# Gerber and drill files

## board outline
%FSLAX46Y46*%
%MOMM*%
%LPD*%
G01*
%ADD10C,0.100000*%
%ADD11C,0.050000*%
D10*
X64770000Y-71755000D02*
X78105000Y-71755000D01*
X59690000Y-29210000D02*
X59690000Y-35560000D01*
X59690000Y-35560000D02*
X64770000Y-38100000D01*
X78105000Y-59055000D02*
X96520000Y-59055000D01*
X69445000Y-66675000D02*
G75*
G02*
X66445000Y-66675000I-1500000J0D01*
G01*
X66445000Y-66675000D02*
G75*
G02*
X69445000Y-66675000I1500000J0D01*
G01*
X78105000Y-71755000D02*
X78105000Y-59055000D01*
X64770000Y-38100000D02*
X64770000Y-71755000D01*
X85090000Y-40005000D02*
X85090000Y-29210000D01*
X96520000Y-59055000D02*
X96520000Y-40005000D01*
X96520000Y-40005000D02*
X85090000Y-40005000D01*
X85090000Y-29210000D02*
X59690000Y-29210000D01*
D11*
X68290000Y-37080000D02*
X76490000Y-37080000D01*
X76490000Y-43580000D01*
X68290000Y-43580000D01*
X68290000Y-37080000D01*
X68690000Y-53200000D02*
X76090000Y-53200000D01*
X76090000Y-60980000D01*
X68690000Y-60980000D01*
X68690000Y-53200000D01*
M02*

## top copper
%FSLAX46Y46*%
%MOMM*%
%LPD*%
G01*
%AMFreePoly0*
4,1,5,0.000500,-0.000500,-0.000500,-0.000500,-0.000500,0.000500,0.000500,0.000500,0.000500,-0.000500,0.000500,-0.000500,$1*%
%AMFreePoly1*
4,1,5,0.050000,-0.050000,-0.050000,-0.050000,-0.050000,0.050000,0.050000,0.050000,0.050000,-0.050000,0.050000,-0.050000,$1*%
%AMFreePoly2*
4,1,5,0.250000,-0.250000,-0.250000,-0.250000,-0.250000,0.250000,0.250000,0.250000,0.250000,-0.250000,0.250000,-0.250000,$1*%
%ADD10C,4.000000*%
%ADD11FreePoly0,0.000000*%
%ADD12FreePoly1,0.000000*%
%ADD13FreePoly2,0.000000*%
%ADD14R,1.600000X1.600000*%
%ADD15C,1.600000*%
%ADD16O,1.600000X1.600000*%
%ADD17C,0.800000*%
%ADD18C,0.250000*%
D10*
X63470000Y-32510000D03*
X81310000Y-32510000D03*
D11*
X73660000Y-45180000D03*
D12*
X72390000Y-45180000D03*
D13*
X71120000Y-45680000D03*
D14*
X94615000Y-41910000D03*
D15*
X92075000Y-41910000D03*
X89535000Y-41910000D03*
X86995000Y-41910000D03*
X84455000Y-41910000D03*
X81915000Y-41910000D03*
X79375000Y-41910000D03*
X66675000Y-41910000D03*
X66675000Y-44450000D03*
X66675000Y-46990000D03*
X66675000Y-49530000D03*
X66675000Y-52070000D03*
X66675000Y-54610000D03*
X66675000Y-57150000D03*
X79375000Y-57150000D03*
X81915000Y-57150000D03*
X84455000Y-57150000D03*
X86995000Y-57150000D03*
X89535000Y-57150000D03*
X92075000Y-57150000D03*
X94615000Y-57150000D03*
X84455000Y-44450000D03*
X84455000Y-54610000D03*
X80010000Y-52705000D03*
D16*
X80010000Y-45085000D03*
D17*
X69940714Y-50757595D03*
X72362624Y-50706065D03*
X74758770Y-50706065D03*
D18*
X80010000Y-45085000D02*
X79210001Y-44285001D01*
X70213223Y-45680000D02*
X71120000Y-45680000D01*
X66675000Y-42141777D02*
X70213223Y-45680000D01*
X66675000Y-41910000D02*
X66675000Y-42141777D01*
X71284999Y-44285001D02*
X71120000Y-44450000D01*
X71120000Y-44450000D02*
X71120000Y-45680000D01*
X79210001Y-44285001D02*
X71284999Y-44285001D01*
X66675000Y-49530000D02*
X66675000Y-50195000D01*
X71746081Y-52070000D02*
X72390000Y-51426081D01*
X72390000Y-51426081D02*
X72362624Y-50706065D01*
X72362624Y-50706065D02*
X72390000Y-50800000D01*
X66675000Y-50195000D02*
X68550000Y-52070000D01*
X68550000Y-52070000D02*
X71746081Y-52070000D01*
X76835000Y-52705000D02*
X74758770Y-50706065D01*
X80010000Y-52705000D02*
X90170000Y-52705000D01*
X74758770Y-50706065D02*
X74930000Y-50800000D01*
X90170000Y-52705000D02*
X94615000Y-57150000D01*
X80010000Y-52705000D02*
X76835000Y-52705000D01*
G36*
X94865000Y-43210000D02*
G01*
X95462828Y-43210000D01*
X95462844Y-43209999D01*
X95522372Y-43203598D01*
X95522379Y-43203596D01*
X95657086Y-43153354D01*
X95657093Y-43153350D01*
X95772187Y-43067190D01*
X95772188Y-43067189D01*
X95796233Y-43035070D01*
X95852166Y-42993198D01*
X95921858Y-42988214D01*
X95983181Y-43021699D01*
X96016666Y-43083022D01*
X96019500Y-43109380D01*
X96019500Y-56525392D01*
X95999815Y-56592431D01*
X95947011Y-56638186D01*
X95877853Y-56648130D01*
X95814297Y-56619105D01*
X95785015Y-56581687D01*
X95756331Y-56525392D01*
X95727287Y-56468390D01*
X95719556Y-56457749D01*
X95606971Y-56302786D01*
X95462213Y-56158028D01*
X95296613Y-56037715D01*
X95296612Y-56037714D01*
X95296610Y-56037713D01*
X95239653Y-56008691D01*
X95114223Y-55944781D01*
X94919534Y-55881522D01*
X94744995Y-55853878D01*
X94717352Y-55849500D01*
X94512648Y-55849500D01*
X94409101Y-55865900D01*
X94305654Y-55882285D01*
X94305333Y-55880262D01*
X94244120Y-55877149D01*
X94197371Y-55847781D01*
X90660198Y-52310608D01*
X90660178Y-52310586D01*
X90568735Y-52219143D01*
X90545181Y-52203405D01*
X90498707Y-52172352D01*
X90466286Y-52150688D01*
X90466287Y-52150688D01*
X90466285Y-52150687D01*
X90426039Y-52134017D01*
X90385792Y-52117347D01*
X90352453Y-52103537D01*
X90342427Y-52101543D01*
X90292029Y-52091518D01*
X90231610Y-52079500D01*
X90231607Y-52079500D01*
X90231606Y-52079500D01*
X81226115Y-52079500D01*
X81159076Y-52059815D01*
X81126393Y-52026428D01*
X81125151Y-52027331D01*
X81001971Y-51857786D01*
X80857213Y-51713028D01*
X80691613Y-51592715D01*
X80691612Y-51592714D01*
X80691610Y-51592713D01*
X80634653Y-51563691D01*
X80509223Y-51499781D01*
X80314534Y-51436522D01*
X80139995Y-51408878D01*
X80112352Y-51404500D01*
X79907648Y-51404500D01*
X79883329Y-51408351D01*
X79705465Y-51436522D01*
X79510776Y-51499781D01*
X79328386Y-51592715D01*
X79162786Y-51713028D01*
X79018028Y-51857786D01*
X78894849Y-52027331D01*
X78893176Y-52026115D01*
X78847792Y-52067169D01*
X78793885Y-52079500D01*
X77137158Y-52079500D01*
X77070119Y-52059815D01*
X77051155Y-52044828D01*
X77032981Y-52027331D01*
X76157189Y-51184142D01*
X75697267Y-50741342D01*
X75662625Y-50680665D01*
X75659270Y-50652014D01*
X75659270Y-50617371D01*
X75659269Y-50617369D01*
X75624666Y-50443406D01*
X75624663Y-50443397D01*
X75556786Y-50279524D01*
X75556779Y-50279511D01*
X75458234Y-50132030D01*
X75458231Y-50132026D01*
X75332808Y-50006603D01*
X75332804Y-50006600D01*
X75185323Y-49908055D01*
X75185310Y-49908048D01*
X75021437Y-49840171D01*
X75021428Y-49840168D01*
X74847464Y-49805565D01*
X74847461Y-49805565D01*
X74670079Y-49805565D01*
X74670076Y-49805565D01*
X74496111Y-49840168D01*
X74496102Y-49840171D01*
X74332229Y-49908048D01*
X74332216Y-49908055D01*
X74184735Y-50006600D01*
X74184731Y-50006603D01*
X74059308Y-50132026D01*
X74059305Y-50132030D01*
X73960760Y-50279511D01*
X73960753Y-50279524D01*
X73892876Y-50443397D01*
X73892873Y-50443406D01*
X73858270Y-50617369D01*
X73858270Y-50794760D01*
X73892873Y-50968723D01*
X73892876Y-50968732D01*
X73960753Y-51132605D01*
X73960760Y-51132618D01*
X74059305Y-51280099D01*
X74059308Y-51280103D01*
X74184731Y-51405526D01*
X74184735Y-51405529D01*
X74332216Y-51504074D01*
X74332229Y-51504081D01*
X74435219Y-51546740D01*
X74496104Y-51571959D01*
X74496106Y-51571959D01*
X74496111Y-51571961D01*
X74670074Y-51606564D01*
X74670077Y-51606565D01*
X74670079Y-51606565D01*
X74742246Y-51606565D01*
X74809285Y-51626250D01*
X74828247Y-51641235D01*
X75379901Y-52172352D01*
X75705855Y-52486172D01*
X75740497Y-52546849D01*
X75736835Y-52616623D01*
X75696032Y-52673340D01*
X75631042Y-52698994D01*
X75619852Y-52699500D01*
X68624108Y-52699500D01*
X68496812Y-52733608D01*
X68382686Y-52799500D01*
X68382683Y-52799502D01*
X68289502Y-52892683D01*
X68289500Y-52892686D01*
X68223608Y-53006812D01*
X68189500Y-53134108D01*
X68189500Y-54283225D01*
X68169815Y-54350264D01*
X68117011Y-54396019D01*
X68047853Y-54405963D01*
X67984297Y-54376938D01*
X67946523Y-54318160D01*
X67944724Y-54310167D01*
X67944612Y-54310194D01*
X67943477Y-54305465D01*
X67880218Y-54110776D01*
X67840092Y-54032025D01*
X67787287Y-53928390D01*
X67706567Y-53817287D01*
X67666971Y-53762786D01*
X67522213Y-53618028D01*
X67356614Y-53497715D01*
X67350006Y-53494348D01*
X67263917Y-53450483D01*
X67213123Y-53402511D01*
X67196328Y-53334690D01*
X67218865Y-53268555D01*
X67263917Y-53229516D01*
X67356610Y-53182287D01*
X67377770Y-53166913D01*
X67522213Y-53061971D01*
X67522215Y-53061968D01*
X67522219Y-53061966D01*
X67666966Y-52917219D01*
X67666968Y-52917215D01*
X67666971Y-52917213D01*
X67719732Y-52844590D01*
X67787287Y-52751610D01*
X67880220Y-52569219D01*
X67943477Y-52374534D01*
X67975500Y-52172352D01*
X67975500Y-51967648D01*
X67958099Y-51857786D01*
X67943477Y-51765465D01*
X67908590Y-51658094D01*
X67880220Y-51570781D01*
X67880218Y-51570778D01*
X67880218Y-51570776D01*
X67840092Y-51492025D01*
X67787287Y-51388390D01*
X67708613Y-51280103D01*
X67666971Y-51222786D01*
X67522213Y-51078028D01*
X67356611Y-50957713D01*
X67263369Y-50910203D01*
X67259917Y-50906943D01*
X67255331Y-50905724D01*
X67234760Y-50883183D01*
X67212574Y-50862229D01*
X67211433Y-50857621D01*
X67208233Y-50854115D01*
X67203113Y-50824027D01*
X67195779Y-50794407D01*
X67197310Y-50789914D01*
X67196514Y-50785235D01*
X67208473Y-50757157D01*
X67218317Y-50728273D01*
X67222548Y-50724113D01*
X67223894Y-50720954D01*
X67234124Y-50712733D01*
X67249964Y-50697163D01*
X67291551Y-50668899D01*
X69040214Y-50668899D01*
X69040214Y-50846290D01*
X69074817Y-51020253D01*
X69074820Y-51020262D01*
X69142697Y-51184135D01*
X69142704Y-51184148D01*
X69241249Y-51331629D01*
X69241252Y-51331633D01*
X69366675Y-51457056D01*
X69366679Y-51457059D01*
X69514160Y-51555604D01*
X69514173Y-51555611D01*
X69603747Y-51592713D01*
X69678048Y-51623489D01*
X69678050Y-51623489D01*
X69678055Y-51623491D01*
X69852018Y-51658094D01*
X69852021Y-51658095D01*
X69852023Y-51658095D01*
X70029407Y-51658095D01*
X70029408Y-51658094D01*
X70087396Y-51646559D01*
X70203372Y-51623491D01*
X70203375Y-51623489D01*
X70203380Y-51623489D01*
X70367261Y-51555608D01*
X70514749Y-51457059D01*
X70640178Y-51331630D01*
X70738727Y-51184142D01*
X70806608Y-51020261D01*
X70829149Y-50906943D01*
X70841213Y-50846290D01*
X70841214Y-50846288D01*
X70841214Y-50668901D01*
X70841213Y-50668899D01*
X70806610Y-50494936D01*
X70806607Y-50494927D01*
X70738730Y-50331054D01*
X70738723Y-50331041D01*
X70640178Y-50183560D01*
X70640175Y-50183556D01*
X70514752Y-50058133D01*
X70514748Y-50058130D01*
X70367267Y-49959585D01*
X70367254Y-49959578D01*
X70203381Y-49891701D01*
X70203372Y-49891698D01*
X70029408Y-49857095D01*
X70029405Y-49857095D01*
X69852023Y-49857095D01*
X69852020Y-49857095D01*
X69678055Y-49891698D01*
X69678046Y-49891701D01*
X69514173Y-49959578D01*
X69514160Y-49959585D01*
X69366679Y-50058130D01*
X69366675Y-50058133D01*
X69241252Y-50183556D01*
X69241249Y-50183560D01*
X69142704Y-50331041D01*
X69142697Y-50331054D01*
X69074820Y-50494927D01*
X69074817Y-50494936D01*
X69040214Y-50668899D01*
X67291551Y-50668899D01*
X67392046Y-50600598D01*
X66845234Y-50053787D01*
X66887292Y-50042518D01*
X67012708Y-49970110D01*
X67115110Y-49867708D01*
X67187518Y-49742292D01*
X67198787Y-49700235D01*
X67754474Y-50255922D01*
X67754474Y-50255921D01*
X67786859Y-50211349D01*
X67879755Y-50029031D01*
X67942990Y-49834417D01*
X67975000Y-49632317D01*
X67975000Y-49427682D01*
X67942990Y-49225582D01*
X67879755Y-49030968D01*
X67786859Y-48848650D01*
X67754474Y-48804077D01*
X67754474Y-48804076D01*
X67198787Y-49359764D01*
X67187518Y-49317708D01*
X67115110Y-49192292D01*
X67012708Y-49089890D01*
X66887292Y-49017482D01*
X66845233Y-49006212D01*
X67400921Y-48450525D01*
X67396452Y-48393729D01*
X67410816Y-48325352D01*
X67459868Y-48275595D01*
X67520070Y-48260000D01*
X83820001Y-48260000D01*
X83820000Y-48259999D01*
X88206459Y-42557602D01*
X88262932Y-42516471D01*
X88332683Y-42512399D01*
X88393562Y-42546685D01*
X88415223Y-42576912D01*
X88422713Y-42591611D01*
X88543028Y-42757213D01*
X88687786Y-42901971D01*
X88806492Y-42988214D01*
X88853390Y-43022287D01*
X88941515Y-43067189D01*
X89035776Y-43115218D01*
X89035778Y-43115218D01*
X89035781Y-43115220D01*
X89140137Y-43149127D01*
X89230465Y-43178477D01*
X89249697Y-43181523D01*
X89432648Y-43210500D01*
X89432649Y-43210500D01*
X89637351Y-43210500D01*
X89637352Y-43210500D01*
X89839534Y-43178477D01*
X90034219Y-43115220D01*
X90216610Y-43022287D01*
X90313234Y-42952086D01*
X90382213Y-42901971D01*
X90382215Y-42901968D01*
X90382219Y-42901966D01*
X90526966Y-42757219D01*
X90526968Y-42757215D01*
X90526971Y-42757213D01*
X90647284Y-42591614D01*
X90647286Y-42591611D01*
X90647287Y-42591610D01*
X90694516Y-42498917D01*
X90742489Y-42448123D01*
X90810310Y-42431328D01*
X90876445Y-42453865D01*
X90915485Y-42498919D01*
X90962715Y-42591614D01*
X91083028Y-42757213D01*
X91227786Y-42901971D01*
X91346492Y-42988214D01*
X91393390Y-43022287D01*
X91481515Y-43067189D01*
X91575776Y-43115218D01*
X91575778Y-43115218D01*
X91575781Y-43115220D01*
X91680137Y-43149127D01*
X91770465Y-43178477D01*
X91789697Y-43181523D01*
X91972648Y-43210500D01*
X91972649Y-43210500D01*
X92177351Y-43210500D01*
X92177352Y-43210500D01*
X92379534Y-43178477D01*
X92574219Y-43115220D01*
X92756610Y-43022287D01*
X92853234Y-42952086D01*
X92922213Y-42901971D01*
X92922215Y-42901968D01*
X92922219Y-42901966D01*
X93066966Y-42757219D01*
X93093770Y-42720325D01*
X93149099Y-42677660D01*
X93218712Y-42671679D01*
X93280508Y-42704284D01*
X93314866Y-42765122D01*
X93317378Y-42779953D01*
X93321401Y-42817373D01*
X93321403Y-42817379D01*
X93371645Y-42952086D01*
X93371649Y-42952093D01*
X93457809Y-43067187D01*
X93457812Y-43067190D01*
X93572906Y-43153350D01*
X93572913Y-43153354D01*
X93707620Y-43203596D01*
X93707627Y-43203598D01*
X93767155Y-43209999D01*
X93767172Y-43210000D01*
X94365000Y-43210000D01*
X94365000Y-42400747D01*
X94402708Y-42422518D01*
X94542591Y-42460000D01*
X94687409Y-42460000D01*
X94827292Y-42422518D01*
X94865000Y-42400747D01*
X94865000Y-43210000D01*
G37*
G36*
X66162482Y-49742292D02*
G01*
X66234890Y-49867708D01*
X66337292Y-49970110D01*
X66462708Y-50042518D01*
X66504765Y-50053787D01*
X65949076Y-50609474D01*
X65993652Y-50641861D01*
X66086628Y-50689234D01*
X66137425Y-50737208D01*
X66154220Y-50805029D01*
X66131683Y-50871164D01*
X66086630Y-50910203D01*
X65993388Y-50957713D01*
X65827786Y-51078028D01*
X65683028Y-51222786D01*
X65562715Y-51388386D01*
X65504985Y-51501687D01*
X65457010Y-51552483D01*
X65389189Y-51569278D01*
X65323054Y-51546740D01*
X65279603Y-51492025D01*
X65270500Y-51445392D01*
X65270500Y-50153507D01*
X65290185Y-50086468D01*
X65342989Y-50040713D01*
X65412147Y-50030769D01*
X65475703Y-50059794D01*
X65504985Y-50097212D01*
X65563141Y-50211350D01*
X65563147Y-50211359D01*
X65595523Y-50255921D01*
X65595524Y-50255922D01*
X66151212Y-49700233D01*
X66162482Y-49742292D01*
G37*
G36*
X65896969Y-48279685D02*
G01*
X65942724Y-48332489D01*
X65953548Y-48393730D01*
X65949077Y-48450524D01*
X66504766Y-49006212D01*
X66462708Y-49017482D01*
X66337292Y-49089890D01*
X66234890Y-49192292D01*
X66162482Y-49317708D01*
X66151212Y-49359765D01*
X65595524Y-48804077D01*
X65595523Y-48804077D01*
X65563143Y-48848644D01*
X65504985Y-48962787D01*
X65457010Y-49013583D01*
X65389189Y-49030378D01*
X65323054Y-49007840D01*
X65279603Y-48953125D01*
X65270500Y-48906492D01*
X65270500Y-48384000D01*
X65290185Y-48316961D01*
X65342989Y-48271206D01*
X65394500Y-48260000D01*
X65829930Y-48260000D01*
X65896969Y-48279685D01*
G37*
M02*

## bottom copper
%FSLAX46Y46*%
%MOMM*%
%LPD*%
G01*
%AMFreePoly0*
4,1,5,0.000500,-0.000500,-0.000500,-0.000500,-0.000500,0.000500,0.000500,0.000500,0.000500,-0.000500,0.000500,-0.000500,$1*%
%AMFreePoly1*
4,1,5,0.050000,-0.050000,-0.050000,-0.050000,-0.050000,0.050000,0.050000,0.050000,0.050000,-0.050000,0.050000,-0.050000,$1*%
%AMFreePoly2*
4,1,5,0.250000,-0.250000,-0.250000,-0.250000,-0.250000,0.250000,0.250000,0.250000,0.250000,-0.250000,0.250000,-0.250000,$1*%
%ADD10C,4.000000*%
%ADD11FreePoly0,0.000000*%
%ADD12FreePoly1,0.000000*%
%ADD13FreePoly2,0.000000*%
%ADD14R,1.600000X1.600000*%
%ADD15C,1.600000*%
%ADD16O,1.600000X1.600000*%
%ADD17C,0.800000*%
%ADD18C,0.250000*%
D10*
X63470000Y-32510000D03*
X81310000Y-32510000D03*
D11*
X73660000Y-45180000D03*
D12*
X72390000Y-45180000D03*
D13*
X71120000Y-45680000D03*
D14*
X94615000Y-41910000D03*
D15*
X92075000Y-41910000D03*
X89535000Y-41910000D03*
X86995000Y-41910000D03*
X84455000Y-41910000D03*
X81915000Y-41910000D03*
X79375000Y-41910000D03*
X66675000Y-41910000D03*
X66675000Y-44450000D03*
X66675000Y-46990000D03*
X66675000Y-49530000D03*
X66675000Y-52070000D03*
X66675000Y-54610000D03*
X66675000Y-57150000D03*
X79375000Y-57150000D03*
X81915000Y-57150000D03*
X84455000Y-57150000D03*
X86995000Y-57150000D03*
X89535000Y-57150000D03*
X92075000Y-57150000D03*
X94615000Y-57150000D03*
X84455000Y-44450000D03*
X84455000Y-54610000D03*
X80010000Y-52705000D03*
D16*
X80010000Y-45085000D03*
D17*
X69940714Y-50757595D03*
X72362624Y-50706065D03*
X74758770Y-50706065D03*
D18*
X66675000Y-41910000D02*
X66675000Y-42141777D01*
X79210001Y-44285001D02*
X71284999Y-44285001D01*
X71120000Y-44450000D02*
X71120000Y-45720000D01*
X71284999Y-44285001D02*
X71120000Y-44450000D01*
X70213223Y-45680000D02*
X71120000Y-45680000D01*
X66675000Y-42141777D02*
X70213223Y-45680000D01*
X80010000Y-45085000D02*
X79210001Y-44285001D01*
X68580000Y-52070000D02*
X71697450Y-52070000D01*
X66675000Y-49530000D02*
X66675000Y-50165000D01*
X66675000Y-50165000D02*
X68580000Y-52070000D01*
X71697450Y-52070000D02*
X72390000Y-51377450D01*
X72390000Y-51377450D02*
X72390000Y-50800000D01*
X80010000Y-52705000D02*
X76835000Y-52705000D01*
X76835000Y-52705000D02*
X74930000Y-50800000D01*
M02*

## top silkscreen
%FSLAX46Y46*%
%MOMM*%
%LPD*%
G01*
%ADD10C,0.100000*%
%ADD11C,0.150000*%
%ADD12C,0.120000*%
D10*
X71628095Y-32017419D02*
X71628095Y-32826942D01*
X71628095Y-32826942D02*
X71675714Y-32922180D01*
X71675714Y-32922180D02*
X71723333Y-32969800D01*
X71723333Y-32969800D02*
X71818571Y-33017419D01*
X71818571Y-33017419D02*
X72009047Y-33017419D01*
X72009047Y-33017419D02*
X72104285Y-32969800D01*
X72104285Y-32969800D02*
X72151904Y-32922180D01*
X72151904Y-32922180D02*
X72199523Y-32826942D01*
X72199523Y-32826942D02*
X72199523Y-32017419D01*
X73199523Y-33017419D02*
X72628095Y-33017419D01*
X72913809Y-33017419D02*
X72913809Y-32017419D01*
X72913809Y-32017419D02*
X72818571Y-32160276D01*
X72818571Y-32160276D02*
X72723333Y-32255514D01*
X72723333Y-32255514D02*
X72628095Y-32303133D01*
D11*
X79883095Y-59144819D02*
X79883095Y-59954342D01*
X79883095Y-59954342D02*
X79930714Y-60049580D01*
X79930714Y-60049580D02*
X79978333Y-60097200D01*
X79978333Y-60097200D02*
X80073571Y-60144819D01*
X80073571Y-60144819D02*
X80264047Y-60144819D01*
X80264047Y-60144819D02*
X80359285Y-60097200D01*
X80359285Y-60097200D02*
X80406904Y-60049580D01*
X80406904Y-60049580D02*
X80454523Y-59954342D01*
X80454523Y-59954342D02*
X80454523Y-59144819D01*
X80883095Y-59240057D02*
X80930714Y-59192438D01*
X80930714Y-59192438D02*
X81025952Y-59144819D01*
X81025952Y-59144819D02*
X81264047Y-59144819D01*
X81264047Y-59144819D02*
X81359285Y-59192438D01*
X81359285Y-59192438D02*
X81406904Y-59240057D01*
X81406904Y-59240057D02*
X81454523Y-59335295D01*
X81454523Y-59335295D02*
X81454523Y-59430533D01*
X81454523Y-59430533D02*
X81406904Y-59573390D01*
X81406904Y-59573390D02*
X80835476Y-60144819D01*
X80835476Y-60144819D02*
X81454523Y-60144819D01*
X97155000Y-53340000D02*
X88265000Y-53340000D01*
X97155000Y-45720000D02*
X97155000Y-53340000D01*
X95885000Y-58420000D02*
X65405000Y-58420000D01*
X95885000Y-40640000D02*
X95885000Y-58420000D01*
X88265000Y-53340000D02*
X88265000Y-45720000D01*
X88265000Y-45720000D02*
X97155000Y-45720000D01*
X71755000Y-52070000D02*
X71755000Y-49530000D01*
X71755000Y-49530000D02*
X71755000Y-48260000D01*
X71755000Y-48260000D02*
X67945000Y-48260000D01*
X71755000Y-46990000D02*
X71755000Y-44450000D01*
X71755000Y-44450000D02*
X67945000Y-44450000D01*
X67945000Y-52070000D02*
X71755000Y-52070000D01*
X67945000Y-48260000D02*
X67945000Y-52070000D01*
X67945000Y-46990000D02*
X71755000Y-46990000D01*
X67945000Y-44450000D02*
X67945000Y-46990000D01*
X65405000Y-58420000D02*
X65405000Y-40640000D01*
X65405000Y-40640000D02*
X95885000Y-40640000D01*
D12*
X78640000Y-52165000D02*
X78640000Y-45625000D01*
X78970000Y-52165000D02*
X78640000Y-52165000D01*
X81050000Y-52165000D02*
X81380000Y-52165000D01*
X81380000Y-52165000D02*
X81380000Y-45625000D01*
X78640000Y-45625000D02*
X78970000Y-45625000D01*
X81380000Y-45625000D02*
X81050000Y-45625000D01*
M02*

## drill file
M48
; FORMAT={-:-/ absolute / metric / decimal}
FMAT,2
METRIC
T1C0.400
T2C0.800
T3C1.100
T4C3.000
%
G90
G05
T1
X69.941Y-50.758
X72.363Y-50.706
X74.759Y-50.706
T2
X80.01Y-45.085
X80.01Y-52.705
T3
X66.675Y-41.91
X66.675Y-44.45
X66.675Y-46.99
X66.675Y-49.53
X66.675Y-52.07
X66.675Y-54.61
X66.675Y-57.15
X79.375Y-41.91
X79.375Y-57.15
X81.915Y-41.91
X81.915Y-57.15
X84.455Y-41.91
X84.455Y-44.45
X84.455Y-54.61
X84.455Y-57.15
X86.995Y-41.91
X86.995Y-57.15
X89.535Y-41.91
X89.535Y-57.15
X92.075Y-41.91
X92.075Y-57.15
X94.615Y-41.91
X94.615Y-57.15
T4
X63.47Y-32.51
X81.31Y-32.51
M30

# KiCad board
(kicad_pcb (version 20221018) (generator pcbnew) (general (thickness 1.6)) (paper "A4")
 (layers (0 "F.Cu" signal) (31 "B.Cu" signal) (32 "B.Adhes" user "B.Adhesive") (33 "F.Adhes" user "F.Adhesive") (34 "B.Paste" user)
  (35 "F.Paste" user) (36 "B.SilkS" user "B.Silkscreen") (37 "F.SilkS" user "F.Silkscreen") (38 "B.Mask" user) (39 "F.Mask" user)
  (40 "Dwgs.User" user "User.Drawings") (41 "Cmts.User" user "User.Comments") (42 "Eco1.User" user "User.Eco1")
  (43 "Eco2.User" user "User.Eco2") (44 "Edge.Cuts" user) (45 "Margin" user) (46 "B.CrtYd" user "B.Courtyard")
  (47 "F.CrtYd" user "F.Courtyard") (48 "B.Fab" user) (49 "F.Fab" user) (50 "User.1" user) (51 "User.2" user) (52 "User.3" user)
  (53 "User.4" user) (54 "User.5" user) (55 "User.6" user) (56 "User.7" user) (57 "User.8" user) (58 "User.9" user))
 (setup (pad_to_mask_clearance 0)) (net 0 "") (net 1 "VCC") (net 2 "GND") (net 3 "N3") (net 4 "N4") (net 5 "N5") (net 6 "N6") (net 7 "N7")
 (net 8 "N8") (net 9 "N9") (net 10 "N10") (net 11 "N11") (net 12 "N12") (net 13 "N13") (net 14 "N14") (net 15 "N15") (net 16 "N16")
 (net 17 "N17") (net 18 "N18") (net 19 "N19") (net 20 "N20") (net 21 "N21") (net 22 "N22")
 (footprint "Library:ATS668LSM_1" (layer "F.Cu") (at 72.39 43.18)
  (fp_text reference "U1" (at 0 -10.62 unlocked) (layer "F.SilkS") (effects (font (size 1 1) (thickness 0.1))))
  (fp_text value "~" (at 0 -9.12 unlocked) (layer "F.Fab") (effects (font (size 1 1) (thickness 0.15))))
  (fp_rect (start -4.1 -6.1) (end 4.1 0.4) (stroke (width 0.05) (type default)) (fill none) (layer "Edge.Cuts"))
  (fp_rect (start -3.7 10.02) (end 3.7 17.8) (stroke (width 0.05) (type default)) (fill none) (layer "Edge.Cuts"))
  (pad "0" thru_hole circle (at -8.92 -10.67) (size 4 4) (drill 3) (layers "*.Cu" "*.Mask"))
  (pad "0" thru_hole circle (at 8.92 -10.67) (size 4 4) (drill 3) (layers "*.Cu" "*.Mask"))
  (pad "1" smd custom (at 1.27 2) (size 0.001 0.001) (layers "F.Cu" "F.Paste" "F.Mask") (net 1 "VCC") (thermal_bridge_angle 45)
   (options (clearance outline) (anchor rect)) (primitives))
  (pad "1" smd custom (at 1.27 2) (size 0.001 0.001) (layers "B.Cu" "B.Paste" "B.Mask") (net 1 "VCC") (thermal_bridge_angle 45)
   (options (clearance outline) (anchor rect)) (primitives))
  (pad "2" smd custom (at 0 2) (size 0.1 0.1) (layers "F.Cu" "F.Paste" "F.Mask") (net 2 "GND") (thermal_bridge_angle 45)
   (options (clearance outline) (anchor rect)) (primitives))
  (pad "2" smd custom (at 0 2) (size 0.1 0.1) (layers "B.Cu" "B.Paste" "B.Mask") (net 2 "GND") (thermal_bridge_angle 45)
   (options (clearance outline) (anchor rect)) (primitives))
  (pad "3" smd custom (at -1.27 2.5) (size 0.5 0.5) (layers "F.Cu" "F.Paste" "F.Mask") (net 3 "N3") (thermal_bridge_angle 45)
   (options (clearance outline) (anchor rect)) (primitives))
  (pad "3" smd custom (at -1.27 2.5) (size 0.5 0.5) (layers "B.Cu" "B.Paste" "B.Mask") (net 3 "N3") (thermal_bridge_angle 45)
   (options (clearance outline) (anchor rect)) (primitives)))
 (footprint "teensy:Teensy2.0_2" (layer "F.Cu") (at 80.645 49.53 180)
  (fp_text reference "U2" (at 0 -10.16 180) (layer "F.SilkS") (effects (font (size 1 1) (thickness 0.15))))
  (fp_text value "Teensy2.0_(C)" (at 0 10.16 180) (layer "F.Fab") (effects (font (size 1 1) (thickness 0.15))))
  (fp_line (start -16.51 -3.81) (end -7.62 -3.81) (stroke (width 0.15) (type solid)) (layer "F.SilkS"))
  (fp_line (start -16.51 3.81) (end -16.51 -3.81) (stroke (width 0.15) (type solid)) (layer "F.SilkS"))
  (fp_line (start -15.24 -8.89) (end 15.24 -8.89) (stroke (width 0.15) (type solid)) (layer "F.SilkS"))
  (fp_line (start -15.24 8.89) (end -15.24 -8.89) (stroke (width 0.15) (type solid)) (layer "F.SilkS"))
  (fp_line (start -7.62 -3.81) (end -7.62 3.81) (stroke (width 0.15) (type solid)) (layer "F.SilkS"))
  (fp_line (start -7.62 3.81) (end -16.51 3.81) (stroke (width 0.15) (type solid)) (layer "F.SilkS"))
  (fp_line (start 8.89 -2.54) (end 8.89 0) (stroke (width 0.15) (type solid)) (layer "F.SilkS"))
  (fp_line (start 8.89 0) (end 8.89 1.27) (stroke (width 0.15) (type solid)) (layer "F.SilkS"))
  (fp_line (start 8.89 1.27) (end 12.7 1.27) (stroke (width 0.15) (type solid)) (layer "F.SilkS"))
  (fp_line (start 8.89 2.54) (end 8.89 5.08) (stroke (width 0.15) (type solid)) (layer "F.SilkS"))
  (fp_line (start 8.89 5.08) (end 12.7 5.08) (stroke (width 0.15) (type solid)) (layer "F.SilkS"))
  (fp_line (start 12.7 -2.54) (end 8.89 -2.54) (stroke (width 0.15) (type solid)) (layer "F.SilkS"))
  (fp_line (start 12.7 1.27) (end 12.7 -2.54) (stroke (width 0.15) (type solid)) (layer "F.SilkS"))
  (fp_line (start 12.7 2.54) (end 8.89 2.54) (stroke (width 0.15) (type solid)) (layer "F.SilkS"))
  (fp_line (start 12.7 5.08) (end 12.7 2.54) (stroke (width 0.15) (type solid)) (layer "F.SilkS"))
  (fp_line (start 15.24 -8.89) (end 15.24 8.89) (stroke (width 0.15) (type solid)) (layer "F.SilkS"))
  (fp_line (start 15.24 8.89) (end -15.24 8.89) (stroke (width 0.15) (type solid)) (layer "F.SilkS"))
  (pad "1" thru_hole rect (at -13.97 7.62 180) (size 1.6 1.6) (drill 1.1) (layers "*.Cu" "*.Mask") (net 2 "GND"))
  (pad "2" thru_hole circle (at -11.43 7.62 180) (size 1.6 1.6) (drill 1.1) (layers "*.Cu" "*.Mask") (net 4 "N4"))
  (pad "3" thru_hole circle (at -8.89 7.62 180) (size 1.6 1.6) (drill 1.1) (layers "*.Cu" "*.Mask") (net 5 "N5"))
  (pad "4" thru_hole circle (at -6.35 7.62 180) (size 1.6 1.6) (drill 1.1) (layers "*.Cu" "*.Mask") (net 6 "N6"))
  (pad "5" thru_hole circle (at -3.81 7.62 180) (size 1.6 1.6) (drill 1.1) (layers "*.Cu" "*.Mask") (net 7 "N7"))
  (pad "6" thru_hole circle (at -1.27 7.62 180) (size 1.6 1.6) (drill 1.1) (layers "*.Cu" "*.Mask") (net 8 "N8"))
  (pad "7" thru_hole circle (at 1.27 7.62 180) (size 1.6 1.6) (drill 1.1) (layers "*.Cu" "*.Mask") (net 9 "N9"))
  (pad "12" thru_hole circle (at 13.97 7.62 180) (size 1.6 1.6) (drill 1.1) (layers "*.Cu" "*.Mask") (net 3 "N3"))
  (pad "13" thru_hole circle (at 13.97 5.08 180) (size 1.6 1.6) (drill 1.1) (layers "*.Cu" "*.Mask") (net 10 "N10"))
  (pad "14" thru_hole circle (at 13.97 2.54 180) (size 1.6 1.6) (drill 1.1) (layers "*.Cu" "*.Mask") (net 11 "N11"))
  (pad "15" thru_hole circle (at 13.97 0 180) (size 1.6 1.6) (drill 1.1) (layers "*.Cu" "*.Mask") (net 2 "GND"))
  (pad "16" thru_hole circle (at 13.97 -2.54 180) (size 1.6 1.6) (drill 1.1) (layers "*.Cu" "*.Mask") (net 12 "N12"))
  (pad "17" thru_hole circle (at 13.97 -5.08 180) (size 1.6 1.6) (drill 1.1) (layers "*.Cu" "*.Mask") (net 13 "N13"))
  (pad "18" thru_hole circle (at 13.97 -7.62 180) (size 1.6 1.6) (drill 1.1) (layers "*.Cu" "*.Mask") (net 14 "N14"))
  (pad "23" thru_hole circle (at 1.27 -7.62 180) (size 1.6 1.6) (drill 1.1) (layers "*.Cu" "*.Mask") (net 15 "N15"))
  (pad "24" thru_hole circle (at -1.27 -7.62 180) (size 1.6 1.6) (drill 1.1) (layers "*.Cu" "*.Mask") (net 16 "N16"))
  (pad "25" thru_hole circle (at -3.81 -7.62 180) (size 1.6 1.6) (drill 1.1) (layers "*.Cu" "*.Mask") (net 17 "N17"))
  (pad "26" thru_hole circle (at -6.35 -7.62 180) (size 1.6 1.6) (drill 1.1) (layers "*.Cu" "*.Mask") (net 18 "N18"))
  (pad "27" thru_hole circle (at -8.89 -7.62 180) (size 1.6 1.6) (drill 1.1) (layers "*.Cu" "*.Mask") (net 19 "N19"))
  (pad "28" thru_hole circle (at -11.43 -7.62 180) (size 1.6 1.6) (drill 1.1) (layers "*.Cu" "*.Mask") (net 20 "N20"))
  (pad "29" thru_hole circle (at -13.97 -7.62 180) (size 1.6 1.6) (drill 1.1) (layers "*.Cu" "*.Mask") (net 1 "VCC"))
  (pad "30" thru_hole circle (at -3.81 5.08 180) (size 1.6 1.6) (drill 1.1) (layers "*.Cu" "*.Mask") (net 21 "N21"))
  (pad "31" thru_hole circle (at -3.81 -5.08 180) (size 1.6 1.6) (drill 1.1) (layers "*.Cu" "*.Mask") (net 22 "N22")))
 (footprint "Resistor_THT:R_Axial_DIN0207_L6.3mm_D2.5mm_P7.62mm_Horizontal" (layer "F.Cu") (at 80.01 52.705 90)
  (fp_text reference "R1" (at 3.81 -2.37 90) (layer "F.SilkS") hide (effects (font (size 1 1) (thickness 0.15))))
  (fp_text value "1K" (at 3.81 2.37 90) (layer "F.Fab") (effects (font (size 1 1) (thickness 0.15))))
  (fp_line (start 0.54 -1.37) (end 7.08 -1.37) (stroke (width 0.12) (type solid)) (layer "F.SilkS"))
  (fp_line (start 0.54 -1.04) (end 0.54 -1.37) (stroke (width 0.12) (type solid)) (layer "F.SilkS"))
  (fp_line (start 0.54 1.04) (end 0.54 1.37) (stroke (width 0.12) (type solid)) (layer "F.SilkS"))
  (fp_line (start 0.54 1.37) (end 7.08 1.37) (stroke (width 0.12) (type solid)) (layer "F.SilkS"))
  (fp_line (start 7.08 -1.37) (end 7.08 -1.04) (stroke (width 0.12) (type solid)) (layer "F.SilkS"))
  (fp_line (start 7.08 1.37) (end 7.08 1.04) (stroke (width 0.12) (type solid)) (layer "F.SilkS"))
  (pad "1" thru_hole circle (at 0 0 90) (size 1.6 1.6) (drill 0.8) (layers "*.Cu" "*.Mask") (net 1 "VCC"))
  (pad "2" thru_hole oval (at 7.62 0 90) (size 1.6 1.6) (drill 0.8) (layers "*.Cu" "*.Mask") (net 3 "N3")))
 (gr_line (start 64.77 71.755) (end 78.105 71.755) (stroke (width 0.1) (type default)) (layer "Edge.Cuts"))
 (gr_line (start 59.69 29.21) (end 59.69 35.56) (stroke (width 0.1) (type default)) (layer "Edge.Cuts"))
 (gr_line (start 59.69 35.56) (end 64.77 38.1) (stroke (width 0.1) (type default)) (layer "Edge.Cuts"))
 (gr_line (start 78.105 59.055) (end 96.52 59.055) (stroke (width 0.1) (type default)) (layer "Edge.Cuts"))
 (gr_circle (center 67.945 66.675) (end 69.445 66.675) (stroke (width 0.1) (type default)) (fill none) (layer "Edge.Cuts"))
 (gr_line (start 78.105 71.755) (end 78.105 59.055) (stroke (width 0.1) (type default)) (layer "Edge.Cuts"))
 (gr_line (start 64.77 38.1) (end 64.77 71.755) (stroke (width 0.1) (type default)) (layer "Edge.Cuts"))
 (gr_line (start 85.09 40.005) (end 85.09 29.21) (stroke (width 0.1) (type default)) (layer "Edge.Cuts"))
 (gr_line (start 96.52 59.055) (end 96.52 40.005) (stroke (width 0.1) (type default)) (layer "Edge.Cuts"))
 (gr_line (start 96.52 40.005) (end 85.09 40.005) (stroke (width 0.1) (type default)) (layer "Edge.Cuts"))
 (gr_line (start 85.09 29.21) (end 59.69 29.21) (stroke (width 0.1) (type default)) (layer "Edge.Cuts"))
 (segment (start 80.01 45.085) (end 79.210001 44.285001) (width 0.25) (layer "F.Cu") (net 3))
 (segment (start 70.213223 45.68) (end 71.12 45.68) (width 0.25) (layer "F.Cu") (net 3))
 (segment (start 66.675 42.141777) (end 70.213223 45.68) (width 0.25) (layer "F.Cu") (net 3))
 (segment (start 66.675 41.91) (end 66.675 42.141777) (width 0.25) (layer "F.Cu") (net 3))
 (segment (start 71.284999 44.285001) (end 71.12 44.45) (width 0.25) (layer "F.Cu") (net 3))
 (segment (start 71.12 44.45) (end 71.12 45.68) (width 0.25) (layer "F.Cu") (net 3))
 (segment (start 79.210001 44.285001) (end 71.284999 44.285001) (width 0.25) (layer "F.Cu") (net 3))
 (via (at 69.940714 50.757595) (size 0.8) (drill 0.4) (layers "F.Cu" "B.Cu") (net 3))
 (segment (start 66.675 41.91) (end 66.675 42.141777) (width 0.25) (layer "B.Cu") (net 3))
 (segment (start 79.210001 44.285001) (end 71.284999 44.285001) (width 0.25) (layer "B.Cu") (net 3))
 (segment (start 71.12 44.45) (end 71.12 45.72) (width 0.25) (layer "B.Cu") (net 3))
 (segment (start 71.284999 44.285001) (end 71.12 44.45) (width 0.25) (layer "B.Cu") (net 3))
 (segment (start 70.213223 45.68) (end 71.12 45.68) (width 0.25) (layer "B.Cu") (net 3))
 (segment (start 66.675 42.141777) (end 70.213223 45.68) (width 0.25) (layer "B.Cu") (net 3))
 (segment (start 80.01 45.085) (end 79.210001 44.285001) (width 0.25) (layer "B.Cu") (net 3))
 (segment (start 66.675 49.53) (end 66.675 50.195) (width 0.25) (layer "F.Cu") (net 2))
 (segment (start 71.746081 52.07) (end 72.39 51.426081) (width 0.25) (layer "F.Cu") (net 2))
 (segment (start 72.39 51.426081) (end 72.362624 50.706065) (width 0.25) (layer "F.Cu") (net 2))
 (segment (start 72.362624 50.706065) (end 72.39 50.8) (width 0.25) (layer "F.Cu") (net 2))
 (segment (start 66.675 50.195) (end 68.55 52.07) (width 0.25) (layer "F.Cu") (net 2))
 (segment (start 68.55 52.07) (end 71.746081 52.07) (width 0.25) (layer "F.Cu") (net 2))
 (via (at 72.362624 50.706065) (size 0.8) (drill 0.4) (layers "F.Cu" "B.Cu") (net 2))
 (segment (start 68.58 52.07) (end 71.69745 52.07) (width 0.25) (layer "B.Cu") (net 2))
 (segment (start 66.675 49.53) (end 66.675 50.165) (width 0.25) (layer "B.Cu") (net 2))
 (segment (start 66.675 50.165) (end 68.58 52.07) (width 0.25) (layer "B.Cu") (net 2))
 (segment (start 71.69745 52.07) (end 72.39 51.37745) (width 0.25) (layer "B.Cu") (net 2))
 (segment (start 72.39 51.37745) (end 72.39 50.8) (width 0.25) (layer "B.Cu") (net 2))
 (segment (start 76.835 52.705) (end 74.75877 50.706065) (width 0.25) (layer "F.Cu") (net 1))
 (segment (start 80.01 52.705) (end 90.17 52.705) (width 0.25) (layer "F.Cu") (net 1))
 (segment (start 74.75877 50.706065) (end 74.93 50.8) (width 0.25) (layer "F.Cu") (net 1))
 (segment (start 90.17 52.705) (end 94.615 57.15) (width 0.25) (layer "F.Cu") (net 1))
 (segment (start 80.01 52.705) (end 76.835 52.705) (width 0.25) (layer "F.Cu") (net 1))
 (via (at 74.75877 50.706065) (size 0.8) (drill 0.4) (layers "F.Cu" "B.Cu") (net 1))
 (segment (start 80.01 52.705) (end 76.835 52.705) (width 0.25) (layer "B.Cu") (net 1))
 (segment (start 76.835 52.705) (end 74.93 50.8) (width 0.25) (layer "B.Cu") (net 1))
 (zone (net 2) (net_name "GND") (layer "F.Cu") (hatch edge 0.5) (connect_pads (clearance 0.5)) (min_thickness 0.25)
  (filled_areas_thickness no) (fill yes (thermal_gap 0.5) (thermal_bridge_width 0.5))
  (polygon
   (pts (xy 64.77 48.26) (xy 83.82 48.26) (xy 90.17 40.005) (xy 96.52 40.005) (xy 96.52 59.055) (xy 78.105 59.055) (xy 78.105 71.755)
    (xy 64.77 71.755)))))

